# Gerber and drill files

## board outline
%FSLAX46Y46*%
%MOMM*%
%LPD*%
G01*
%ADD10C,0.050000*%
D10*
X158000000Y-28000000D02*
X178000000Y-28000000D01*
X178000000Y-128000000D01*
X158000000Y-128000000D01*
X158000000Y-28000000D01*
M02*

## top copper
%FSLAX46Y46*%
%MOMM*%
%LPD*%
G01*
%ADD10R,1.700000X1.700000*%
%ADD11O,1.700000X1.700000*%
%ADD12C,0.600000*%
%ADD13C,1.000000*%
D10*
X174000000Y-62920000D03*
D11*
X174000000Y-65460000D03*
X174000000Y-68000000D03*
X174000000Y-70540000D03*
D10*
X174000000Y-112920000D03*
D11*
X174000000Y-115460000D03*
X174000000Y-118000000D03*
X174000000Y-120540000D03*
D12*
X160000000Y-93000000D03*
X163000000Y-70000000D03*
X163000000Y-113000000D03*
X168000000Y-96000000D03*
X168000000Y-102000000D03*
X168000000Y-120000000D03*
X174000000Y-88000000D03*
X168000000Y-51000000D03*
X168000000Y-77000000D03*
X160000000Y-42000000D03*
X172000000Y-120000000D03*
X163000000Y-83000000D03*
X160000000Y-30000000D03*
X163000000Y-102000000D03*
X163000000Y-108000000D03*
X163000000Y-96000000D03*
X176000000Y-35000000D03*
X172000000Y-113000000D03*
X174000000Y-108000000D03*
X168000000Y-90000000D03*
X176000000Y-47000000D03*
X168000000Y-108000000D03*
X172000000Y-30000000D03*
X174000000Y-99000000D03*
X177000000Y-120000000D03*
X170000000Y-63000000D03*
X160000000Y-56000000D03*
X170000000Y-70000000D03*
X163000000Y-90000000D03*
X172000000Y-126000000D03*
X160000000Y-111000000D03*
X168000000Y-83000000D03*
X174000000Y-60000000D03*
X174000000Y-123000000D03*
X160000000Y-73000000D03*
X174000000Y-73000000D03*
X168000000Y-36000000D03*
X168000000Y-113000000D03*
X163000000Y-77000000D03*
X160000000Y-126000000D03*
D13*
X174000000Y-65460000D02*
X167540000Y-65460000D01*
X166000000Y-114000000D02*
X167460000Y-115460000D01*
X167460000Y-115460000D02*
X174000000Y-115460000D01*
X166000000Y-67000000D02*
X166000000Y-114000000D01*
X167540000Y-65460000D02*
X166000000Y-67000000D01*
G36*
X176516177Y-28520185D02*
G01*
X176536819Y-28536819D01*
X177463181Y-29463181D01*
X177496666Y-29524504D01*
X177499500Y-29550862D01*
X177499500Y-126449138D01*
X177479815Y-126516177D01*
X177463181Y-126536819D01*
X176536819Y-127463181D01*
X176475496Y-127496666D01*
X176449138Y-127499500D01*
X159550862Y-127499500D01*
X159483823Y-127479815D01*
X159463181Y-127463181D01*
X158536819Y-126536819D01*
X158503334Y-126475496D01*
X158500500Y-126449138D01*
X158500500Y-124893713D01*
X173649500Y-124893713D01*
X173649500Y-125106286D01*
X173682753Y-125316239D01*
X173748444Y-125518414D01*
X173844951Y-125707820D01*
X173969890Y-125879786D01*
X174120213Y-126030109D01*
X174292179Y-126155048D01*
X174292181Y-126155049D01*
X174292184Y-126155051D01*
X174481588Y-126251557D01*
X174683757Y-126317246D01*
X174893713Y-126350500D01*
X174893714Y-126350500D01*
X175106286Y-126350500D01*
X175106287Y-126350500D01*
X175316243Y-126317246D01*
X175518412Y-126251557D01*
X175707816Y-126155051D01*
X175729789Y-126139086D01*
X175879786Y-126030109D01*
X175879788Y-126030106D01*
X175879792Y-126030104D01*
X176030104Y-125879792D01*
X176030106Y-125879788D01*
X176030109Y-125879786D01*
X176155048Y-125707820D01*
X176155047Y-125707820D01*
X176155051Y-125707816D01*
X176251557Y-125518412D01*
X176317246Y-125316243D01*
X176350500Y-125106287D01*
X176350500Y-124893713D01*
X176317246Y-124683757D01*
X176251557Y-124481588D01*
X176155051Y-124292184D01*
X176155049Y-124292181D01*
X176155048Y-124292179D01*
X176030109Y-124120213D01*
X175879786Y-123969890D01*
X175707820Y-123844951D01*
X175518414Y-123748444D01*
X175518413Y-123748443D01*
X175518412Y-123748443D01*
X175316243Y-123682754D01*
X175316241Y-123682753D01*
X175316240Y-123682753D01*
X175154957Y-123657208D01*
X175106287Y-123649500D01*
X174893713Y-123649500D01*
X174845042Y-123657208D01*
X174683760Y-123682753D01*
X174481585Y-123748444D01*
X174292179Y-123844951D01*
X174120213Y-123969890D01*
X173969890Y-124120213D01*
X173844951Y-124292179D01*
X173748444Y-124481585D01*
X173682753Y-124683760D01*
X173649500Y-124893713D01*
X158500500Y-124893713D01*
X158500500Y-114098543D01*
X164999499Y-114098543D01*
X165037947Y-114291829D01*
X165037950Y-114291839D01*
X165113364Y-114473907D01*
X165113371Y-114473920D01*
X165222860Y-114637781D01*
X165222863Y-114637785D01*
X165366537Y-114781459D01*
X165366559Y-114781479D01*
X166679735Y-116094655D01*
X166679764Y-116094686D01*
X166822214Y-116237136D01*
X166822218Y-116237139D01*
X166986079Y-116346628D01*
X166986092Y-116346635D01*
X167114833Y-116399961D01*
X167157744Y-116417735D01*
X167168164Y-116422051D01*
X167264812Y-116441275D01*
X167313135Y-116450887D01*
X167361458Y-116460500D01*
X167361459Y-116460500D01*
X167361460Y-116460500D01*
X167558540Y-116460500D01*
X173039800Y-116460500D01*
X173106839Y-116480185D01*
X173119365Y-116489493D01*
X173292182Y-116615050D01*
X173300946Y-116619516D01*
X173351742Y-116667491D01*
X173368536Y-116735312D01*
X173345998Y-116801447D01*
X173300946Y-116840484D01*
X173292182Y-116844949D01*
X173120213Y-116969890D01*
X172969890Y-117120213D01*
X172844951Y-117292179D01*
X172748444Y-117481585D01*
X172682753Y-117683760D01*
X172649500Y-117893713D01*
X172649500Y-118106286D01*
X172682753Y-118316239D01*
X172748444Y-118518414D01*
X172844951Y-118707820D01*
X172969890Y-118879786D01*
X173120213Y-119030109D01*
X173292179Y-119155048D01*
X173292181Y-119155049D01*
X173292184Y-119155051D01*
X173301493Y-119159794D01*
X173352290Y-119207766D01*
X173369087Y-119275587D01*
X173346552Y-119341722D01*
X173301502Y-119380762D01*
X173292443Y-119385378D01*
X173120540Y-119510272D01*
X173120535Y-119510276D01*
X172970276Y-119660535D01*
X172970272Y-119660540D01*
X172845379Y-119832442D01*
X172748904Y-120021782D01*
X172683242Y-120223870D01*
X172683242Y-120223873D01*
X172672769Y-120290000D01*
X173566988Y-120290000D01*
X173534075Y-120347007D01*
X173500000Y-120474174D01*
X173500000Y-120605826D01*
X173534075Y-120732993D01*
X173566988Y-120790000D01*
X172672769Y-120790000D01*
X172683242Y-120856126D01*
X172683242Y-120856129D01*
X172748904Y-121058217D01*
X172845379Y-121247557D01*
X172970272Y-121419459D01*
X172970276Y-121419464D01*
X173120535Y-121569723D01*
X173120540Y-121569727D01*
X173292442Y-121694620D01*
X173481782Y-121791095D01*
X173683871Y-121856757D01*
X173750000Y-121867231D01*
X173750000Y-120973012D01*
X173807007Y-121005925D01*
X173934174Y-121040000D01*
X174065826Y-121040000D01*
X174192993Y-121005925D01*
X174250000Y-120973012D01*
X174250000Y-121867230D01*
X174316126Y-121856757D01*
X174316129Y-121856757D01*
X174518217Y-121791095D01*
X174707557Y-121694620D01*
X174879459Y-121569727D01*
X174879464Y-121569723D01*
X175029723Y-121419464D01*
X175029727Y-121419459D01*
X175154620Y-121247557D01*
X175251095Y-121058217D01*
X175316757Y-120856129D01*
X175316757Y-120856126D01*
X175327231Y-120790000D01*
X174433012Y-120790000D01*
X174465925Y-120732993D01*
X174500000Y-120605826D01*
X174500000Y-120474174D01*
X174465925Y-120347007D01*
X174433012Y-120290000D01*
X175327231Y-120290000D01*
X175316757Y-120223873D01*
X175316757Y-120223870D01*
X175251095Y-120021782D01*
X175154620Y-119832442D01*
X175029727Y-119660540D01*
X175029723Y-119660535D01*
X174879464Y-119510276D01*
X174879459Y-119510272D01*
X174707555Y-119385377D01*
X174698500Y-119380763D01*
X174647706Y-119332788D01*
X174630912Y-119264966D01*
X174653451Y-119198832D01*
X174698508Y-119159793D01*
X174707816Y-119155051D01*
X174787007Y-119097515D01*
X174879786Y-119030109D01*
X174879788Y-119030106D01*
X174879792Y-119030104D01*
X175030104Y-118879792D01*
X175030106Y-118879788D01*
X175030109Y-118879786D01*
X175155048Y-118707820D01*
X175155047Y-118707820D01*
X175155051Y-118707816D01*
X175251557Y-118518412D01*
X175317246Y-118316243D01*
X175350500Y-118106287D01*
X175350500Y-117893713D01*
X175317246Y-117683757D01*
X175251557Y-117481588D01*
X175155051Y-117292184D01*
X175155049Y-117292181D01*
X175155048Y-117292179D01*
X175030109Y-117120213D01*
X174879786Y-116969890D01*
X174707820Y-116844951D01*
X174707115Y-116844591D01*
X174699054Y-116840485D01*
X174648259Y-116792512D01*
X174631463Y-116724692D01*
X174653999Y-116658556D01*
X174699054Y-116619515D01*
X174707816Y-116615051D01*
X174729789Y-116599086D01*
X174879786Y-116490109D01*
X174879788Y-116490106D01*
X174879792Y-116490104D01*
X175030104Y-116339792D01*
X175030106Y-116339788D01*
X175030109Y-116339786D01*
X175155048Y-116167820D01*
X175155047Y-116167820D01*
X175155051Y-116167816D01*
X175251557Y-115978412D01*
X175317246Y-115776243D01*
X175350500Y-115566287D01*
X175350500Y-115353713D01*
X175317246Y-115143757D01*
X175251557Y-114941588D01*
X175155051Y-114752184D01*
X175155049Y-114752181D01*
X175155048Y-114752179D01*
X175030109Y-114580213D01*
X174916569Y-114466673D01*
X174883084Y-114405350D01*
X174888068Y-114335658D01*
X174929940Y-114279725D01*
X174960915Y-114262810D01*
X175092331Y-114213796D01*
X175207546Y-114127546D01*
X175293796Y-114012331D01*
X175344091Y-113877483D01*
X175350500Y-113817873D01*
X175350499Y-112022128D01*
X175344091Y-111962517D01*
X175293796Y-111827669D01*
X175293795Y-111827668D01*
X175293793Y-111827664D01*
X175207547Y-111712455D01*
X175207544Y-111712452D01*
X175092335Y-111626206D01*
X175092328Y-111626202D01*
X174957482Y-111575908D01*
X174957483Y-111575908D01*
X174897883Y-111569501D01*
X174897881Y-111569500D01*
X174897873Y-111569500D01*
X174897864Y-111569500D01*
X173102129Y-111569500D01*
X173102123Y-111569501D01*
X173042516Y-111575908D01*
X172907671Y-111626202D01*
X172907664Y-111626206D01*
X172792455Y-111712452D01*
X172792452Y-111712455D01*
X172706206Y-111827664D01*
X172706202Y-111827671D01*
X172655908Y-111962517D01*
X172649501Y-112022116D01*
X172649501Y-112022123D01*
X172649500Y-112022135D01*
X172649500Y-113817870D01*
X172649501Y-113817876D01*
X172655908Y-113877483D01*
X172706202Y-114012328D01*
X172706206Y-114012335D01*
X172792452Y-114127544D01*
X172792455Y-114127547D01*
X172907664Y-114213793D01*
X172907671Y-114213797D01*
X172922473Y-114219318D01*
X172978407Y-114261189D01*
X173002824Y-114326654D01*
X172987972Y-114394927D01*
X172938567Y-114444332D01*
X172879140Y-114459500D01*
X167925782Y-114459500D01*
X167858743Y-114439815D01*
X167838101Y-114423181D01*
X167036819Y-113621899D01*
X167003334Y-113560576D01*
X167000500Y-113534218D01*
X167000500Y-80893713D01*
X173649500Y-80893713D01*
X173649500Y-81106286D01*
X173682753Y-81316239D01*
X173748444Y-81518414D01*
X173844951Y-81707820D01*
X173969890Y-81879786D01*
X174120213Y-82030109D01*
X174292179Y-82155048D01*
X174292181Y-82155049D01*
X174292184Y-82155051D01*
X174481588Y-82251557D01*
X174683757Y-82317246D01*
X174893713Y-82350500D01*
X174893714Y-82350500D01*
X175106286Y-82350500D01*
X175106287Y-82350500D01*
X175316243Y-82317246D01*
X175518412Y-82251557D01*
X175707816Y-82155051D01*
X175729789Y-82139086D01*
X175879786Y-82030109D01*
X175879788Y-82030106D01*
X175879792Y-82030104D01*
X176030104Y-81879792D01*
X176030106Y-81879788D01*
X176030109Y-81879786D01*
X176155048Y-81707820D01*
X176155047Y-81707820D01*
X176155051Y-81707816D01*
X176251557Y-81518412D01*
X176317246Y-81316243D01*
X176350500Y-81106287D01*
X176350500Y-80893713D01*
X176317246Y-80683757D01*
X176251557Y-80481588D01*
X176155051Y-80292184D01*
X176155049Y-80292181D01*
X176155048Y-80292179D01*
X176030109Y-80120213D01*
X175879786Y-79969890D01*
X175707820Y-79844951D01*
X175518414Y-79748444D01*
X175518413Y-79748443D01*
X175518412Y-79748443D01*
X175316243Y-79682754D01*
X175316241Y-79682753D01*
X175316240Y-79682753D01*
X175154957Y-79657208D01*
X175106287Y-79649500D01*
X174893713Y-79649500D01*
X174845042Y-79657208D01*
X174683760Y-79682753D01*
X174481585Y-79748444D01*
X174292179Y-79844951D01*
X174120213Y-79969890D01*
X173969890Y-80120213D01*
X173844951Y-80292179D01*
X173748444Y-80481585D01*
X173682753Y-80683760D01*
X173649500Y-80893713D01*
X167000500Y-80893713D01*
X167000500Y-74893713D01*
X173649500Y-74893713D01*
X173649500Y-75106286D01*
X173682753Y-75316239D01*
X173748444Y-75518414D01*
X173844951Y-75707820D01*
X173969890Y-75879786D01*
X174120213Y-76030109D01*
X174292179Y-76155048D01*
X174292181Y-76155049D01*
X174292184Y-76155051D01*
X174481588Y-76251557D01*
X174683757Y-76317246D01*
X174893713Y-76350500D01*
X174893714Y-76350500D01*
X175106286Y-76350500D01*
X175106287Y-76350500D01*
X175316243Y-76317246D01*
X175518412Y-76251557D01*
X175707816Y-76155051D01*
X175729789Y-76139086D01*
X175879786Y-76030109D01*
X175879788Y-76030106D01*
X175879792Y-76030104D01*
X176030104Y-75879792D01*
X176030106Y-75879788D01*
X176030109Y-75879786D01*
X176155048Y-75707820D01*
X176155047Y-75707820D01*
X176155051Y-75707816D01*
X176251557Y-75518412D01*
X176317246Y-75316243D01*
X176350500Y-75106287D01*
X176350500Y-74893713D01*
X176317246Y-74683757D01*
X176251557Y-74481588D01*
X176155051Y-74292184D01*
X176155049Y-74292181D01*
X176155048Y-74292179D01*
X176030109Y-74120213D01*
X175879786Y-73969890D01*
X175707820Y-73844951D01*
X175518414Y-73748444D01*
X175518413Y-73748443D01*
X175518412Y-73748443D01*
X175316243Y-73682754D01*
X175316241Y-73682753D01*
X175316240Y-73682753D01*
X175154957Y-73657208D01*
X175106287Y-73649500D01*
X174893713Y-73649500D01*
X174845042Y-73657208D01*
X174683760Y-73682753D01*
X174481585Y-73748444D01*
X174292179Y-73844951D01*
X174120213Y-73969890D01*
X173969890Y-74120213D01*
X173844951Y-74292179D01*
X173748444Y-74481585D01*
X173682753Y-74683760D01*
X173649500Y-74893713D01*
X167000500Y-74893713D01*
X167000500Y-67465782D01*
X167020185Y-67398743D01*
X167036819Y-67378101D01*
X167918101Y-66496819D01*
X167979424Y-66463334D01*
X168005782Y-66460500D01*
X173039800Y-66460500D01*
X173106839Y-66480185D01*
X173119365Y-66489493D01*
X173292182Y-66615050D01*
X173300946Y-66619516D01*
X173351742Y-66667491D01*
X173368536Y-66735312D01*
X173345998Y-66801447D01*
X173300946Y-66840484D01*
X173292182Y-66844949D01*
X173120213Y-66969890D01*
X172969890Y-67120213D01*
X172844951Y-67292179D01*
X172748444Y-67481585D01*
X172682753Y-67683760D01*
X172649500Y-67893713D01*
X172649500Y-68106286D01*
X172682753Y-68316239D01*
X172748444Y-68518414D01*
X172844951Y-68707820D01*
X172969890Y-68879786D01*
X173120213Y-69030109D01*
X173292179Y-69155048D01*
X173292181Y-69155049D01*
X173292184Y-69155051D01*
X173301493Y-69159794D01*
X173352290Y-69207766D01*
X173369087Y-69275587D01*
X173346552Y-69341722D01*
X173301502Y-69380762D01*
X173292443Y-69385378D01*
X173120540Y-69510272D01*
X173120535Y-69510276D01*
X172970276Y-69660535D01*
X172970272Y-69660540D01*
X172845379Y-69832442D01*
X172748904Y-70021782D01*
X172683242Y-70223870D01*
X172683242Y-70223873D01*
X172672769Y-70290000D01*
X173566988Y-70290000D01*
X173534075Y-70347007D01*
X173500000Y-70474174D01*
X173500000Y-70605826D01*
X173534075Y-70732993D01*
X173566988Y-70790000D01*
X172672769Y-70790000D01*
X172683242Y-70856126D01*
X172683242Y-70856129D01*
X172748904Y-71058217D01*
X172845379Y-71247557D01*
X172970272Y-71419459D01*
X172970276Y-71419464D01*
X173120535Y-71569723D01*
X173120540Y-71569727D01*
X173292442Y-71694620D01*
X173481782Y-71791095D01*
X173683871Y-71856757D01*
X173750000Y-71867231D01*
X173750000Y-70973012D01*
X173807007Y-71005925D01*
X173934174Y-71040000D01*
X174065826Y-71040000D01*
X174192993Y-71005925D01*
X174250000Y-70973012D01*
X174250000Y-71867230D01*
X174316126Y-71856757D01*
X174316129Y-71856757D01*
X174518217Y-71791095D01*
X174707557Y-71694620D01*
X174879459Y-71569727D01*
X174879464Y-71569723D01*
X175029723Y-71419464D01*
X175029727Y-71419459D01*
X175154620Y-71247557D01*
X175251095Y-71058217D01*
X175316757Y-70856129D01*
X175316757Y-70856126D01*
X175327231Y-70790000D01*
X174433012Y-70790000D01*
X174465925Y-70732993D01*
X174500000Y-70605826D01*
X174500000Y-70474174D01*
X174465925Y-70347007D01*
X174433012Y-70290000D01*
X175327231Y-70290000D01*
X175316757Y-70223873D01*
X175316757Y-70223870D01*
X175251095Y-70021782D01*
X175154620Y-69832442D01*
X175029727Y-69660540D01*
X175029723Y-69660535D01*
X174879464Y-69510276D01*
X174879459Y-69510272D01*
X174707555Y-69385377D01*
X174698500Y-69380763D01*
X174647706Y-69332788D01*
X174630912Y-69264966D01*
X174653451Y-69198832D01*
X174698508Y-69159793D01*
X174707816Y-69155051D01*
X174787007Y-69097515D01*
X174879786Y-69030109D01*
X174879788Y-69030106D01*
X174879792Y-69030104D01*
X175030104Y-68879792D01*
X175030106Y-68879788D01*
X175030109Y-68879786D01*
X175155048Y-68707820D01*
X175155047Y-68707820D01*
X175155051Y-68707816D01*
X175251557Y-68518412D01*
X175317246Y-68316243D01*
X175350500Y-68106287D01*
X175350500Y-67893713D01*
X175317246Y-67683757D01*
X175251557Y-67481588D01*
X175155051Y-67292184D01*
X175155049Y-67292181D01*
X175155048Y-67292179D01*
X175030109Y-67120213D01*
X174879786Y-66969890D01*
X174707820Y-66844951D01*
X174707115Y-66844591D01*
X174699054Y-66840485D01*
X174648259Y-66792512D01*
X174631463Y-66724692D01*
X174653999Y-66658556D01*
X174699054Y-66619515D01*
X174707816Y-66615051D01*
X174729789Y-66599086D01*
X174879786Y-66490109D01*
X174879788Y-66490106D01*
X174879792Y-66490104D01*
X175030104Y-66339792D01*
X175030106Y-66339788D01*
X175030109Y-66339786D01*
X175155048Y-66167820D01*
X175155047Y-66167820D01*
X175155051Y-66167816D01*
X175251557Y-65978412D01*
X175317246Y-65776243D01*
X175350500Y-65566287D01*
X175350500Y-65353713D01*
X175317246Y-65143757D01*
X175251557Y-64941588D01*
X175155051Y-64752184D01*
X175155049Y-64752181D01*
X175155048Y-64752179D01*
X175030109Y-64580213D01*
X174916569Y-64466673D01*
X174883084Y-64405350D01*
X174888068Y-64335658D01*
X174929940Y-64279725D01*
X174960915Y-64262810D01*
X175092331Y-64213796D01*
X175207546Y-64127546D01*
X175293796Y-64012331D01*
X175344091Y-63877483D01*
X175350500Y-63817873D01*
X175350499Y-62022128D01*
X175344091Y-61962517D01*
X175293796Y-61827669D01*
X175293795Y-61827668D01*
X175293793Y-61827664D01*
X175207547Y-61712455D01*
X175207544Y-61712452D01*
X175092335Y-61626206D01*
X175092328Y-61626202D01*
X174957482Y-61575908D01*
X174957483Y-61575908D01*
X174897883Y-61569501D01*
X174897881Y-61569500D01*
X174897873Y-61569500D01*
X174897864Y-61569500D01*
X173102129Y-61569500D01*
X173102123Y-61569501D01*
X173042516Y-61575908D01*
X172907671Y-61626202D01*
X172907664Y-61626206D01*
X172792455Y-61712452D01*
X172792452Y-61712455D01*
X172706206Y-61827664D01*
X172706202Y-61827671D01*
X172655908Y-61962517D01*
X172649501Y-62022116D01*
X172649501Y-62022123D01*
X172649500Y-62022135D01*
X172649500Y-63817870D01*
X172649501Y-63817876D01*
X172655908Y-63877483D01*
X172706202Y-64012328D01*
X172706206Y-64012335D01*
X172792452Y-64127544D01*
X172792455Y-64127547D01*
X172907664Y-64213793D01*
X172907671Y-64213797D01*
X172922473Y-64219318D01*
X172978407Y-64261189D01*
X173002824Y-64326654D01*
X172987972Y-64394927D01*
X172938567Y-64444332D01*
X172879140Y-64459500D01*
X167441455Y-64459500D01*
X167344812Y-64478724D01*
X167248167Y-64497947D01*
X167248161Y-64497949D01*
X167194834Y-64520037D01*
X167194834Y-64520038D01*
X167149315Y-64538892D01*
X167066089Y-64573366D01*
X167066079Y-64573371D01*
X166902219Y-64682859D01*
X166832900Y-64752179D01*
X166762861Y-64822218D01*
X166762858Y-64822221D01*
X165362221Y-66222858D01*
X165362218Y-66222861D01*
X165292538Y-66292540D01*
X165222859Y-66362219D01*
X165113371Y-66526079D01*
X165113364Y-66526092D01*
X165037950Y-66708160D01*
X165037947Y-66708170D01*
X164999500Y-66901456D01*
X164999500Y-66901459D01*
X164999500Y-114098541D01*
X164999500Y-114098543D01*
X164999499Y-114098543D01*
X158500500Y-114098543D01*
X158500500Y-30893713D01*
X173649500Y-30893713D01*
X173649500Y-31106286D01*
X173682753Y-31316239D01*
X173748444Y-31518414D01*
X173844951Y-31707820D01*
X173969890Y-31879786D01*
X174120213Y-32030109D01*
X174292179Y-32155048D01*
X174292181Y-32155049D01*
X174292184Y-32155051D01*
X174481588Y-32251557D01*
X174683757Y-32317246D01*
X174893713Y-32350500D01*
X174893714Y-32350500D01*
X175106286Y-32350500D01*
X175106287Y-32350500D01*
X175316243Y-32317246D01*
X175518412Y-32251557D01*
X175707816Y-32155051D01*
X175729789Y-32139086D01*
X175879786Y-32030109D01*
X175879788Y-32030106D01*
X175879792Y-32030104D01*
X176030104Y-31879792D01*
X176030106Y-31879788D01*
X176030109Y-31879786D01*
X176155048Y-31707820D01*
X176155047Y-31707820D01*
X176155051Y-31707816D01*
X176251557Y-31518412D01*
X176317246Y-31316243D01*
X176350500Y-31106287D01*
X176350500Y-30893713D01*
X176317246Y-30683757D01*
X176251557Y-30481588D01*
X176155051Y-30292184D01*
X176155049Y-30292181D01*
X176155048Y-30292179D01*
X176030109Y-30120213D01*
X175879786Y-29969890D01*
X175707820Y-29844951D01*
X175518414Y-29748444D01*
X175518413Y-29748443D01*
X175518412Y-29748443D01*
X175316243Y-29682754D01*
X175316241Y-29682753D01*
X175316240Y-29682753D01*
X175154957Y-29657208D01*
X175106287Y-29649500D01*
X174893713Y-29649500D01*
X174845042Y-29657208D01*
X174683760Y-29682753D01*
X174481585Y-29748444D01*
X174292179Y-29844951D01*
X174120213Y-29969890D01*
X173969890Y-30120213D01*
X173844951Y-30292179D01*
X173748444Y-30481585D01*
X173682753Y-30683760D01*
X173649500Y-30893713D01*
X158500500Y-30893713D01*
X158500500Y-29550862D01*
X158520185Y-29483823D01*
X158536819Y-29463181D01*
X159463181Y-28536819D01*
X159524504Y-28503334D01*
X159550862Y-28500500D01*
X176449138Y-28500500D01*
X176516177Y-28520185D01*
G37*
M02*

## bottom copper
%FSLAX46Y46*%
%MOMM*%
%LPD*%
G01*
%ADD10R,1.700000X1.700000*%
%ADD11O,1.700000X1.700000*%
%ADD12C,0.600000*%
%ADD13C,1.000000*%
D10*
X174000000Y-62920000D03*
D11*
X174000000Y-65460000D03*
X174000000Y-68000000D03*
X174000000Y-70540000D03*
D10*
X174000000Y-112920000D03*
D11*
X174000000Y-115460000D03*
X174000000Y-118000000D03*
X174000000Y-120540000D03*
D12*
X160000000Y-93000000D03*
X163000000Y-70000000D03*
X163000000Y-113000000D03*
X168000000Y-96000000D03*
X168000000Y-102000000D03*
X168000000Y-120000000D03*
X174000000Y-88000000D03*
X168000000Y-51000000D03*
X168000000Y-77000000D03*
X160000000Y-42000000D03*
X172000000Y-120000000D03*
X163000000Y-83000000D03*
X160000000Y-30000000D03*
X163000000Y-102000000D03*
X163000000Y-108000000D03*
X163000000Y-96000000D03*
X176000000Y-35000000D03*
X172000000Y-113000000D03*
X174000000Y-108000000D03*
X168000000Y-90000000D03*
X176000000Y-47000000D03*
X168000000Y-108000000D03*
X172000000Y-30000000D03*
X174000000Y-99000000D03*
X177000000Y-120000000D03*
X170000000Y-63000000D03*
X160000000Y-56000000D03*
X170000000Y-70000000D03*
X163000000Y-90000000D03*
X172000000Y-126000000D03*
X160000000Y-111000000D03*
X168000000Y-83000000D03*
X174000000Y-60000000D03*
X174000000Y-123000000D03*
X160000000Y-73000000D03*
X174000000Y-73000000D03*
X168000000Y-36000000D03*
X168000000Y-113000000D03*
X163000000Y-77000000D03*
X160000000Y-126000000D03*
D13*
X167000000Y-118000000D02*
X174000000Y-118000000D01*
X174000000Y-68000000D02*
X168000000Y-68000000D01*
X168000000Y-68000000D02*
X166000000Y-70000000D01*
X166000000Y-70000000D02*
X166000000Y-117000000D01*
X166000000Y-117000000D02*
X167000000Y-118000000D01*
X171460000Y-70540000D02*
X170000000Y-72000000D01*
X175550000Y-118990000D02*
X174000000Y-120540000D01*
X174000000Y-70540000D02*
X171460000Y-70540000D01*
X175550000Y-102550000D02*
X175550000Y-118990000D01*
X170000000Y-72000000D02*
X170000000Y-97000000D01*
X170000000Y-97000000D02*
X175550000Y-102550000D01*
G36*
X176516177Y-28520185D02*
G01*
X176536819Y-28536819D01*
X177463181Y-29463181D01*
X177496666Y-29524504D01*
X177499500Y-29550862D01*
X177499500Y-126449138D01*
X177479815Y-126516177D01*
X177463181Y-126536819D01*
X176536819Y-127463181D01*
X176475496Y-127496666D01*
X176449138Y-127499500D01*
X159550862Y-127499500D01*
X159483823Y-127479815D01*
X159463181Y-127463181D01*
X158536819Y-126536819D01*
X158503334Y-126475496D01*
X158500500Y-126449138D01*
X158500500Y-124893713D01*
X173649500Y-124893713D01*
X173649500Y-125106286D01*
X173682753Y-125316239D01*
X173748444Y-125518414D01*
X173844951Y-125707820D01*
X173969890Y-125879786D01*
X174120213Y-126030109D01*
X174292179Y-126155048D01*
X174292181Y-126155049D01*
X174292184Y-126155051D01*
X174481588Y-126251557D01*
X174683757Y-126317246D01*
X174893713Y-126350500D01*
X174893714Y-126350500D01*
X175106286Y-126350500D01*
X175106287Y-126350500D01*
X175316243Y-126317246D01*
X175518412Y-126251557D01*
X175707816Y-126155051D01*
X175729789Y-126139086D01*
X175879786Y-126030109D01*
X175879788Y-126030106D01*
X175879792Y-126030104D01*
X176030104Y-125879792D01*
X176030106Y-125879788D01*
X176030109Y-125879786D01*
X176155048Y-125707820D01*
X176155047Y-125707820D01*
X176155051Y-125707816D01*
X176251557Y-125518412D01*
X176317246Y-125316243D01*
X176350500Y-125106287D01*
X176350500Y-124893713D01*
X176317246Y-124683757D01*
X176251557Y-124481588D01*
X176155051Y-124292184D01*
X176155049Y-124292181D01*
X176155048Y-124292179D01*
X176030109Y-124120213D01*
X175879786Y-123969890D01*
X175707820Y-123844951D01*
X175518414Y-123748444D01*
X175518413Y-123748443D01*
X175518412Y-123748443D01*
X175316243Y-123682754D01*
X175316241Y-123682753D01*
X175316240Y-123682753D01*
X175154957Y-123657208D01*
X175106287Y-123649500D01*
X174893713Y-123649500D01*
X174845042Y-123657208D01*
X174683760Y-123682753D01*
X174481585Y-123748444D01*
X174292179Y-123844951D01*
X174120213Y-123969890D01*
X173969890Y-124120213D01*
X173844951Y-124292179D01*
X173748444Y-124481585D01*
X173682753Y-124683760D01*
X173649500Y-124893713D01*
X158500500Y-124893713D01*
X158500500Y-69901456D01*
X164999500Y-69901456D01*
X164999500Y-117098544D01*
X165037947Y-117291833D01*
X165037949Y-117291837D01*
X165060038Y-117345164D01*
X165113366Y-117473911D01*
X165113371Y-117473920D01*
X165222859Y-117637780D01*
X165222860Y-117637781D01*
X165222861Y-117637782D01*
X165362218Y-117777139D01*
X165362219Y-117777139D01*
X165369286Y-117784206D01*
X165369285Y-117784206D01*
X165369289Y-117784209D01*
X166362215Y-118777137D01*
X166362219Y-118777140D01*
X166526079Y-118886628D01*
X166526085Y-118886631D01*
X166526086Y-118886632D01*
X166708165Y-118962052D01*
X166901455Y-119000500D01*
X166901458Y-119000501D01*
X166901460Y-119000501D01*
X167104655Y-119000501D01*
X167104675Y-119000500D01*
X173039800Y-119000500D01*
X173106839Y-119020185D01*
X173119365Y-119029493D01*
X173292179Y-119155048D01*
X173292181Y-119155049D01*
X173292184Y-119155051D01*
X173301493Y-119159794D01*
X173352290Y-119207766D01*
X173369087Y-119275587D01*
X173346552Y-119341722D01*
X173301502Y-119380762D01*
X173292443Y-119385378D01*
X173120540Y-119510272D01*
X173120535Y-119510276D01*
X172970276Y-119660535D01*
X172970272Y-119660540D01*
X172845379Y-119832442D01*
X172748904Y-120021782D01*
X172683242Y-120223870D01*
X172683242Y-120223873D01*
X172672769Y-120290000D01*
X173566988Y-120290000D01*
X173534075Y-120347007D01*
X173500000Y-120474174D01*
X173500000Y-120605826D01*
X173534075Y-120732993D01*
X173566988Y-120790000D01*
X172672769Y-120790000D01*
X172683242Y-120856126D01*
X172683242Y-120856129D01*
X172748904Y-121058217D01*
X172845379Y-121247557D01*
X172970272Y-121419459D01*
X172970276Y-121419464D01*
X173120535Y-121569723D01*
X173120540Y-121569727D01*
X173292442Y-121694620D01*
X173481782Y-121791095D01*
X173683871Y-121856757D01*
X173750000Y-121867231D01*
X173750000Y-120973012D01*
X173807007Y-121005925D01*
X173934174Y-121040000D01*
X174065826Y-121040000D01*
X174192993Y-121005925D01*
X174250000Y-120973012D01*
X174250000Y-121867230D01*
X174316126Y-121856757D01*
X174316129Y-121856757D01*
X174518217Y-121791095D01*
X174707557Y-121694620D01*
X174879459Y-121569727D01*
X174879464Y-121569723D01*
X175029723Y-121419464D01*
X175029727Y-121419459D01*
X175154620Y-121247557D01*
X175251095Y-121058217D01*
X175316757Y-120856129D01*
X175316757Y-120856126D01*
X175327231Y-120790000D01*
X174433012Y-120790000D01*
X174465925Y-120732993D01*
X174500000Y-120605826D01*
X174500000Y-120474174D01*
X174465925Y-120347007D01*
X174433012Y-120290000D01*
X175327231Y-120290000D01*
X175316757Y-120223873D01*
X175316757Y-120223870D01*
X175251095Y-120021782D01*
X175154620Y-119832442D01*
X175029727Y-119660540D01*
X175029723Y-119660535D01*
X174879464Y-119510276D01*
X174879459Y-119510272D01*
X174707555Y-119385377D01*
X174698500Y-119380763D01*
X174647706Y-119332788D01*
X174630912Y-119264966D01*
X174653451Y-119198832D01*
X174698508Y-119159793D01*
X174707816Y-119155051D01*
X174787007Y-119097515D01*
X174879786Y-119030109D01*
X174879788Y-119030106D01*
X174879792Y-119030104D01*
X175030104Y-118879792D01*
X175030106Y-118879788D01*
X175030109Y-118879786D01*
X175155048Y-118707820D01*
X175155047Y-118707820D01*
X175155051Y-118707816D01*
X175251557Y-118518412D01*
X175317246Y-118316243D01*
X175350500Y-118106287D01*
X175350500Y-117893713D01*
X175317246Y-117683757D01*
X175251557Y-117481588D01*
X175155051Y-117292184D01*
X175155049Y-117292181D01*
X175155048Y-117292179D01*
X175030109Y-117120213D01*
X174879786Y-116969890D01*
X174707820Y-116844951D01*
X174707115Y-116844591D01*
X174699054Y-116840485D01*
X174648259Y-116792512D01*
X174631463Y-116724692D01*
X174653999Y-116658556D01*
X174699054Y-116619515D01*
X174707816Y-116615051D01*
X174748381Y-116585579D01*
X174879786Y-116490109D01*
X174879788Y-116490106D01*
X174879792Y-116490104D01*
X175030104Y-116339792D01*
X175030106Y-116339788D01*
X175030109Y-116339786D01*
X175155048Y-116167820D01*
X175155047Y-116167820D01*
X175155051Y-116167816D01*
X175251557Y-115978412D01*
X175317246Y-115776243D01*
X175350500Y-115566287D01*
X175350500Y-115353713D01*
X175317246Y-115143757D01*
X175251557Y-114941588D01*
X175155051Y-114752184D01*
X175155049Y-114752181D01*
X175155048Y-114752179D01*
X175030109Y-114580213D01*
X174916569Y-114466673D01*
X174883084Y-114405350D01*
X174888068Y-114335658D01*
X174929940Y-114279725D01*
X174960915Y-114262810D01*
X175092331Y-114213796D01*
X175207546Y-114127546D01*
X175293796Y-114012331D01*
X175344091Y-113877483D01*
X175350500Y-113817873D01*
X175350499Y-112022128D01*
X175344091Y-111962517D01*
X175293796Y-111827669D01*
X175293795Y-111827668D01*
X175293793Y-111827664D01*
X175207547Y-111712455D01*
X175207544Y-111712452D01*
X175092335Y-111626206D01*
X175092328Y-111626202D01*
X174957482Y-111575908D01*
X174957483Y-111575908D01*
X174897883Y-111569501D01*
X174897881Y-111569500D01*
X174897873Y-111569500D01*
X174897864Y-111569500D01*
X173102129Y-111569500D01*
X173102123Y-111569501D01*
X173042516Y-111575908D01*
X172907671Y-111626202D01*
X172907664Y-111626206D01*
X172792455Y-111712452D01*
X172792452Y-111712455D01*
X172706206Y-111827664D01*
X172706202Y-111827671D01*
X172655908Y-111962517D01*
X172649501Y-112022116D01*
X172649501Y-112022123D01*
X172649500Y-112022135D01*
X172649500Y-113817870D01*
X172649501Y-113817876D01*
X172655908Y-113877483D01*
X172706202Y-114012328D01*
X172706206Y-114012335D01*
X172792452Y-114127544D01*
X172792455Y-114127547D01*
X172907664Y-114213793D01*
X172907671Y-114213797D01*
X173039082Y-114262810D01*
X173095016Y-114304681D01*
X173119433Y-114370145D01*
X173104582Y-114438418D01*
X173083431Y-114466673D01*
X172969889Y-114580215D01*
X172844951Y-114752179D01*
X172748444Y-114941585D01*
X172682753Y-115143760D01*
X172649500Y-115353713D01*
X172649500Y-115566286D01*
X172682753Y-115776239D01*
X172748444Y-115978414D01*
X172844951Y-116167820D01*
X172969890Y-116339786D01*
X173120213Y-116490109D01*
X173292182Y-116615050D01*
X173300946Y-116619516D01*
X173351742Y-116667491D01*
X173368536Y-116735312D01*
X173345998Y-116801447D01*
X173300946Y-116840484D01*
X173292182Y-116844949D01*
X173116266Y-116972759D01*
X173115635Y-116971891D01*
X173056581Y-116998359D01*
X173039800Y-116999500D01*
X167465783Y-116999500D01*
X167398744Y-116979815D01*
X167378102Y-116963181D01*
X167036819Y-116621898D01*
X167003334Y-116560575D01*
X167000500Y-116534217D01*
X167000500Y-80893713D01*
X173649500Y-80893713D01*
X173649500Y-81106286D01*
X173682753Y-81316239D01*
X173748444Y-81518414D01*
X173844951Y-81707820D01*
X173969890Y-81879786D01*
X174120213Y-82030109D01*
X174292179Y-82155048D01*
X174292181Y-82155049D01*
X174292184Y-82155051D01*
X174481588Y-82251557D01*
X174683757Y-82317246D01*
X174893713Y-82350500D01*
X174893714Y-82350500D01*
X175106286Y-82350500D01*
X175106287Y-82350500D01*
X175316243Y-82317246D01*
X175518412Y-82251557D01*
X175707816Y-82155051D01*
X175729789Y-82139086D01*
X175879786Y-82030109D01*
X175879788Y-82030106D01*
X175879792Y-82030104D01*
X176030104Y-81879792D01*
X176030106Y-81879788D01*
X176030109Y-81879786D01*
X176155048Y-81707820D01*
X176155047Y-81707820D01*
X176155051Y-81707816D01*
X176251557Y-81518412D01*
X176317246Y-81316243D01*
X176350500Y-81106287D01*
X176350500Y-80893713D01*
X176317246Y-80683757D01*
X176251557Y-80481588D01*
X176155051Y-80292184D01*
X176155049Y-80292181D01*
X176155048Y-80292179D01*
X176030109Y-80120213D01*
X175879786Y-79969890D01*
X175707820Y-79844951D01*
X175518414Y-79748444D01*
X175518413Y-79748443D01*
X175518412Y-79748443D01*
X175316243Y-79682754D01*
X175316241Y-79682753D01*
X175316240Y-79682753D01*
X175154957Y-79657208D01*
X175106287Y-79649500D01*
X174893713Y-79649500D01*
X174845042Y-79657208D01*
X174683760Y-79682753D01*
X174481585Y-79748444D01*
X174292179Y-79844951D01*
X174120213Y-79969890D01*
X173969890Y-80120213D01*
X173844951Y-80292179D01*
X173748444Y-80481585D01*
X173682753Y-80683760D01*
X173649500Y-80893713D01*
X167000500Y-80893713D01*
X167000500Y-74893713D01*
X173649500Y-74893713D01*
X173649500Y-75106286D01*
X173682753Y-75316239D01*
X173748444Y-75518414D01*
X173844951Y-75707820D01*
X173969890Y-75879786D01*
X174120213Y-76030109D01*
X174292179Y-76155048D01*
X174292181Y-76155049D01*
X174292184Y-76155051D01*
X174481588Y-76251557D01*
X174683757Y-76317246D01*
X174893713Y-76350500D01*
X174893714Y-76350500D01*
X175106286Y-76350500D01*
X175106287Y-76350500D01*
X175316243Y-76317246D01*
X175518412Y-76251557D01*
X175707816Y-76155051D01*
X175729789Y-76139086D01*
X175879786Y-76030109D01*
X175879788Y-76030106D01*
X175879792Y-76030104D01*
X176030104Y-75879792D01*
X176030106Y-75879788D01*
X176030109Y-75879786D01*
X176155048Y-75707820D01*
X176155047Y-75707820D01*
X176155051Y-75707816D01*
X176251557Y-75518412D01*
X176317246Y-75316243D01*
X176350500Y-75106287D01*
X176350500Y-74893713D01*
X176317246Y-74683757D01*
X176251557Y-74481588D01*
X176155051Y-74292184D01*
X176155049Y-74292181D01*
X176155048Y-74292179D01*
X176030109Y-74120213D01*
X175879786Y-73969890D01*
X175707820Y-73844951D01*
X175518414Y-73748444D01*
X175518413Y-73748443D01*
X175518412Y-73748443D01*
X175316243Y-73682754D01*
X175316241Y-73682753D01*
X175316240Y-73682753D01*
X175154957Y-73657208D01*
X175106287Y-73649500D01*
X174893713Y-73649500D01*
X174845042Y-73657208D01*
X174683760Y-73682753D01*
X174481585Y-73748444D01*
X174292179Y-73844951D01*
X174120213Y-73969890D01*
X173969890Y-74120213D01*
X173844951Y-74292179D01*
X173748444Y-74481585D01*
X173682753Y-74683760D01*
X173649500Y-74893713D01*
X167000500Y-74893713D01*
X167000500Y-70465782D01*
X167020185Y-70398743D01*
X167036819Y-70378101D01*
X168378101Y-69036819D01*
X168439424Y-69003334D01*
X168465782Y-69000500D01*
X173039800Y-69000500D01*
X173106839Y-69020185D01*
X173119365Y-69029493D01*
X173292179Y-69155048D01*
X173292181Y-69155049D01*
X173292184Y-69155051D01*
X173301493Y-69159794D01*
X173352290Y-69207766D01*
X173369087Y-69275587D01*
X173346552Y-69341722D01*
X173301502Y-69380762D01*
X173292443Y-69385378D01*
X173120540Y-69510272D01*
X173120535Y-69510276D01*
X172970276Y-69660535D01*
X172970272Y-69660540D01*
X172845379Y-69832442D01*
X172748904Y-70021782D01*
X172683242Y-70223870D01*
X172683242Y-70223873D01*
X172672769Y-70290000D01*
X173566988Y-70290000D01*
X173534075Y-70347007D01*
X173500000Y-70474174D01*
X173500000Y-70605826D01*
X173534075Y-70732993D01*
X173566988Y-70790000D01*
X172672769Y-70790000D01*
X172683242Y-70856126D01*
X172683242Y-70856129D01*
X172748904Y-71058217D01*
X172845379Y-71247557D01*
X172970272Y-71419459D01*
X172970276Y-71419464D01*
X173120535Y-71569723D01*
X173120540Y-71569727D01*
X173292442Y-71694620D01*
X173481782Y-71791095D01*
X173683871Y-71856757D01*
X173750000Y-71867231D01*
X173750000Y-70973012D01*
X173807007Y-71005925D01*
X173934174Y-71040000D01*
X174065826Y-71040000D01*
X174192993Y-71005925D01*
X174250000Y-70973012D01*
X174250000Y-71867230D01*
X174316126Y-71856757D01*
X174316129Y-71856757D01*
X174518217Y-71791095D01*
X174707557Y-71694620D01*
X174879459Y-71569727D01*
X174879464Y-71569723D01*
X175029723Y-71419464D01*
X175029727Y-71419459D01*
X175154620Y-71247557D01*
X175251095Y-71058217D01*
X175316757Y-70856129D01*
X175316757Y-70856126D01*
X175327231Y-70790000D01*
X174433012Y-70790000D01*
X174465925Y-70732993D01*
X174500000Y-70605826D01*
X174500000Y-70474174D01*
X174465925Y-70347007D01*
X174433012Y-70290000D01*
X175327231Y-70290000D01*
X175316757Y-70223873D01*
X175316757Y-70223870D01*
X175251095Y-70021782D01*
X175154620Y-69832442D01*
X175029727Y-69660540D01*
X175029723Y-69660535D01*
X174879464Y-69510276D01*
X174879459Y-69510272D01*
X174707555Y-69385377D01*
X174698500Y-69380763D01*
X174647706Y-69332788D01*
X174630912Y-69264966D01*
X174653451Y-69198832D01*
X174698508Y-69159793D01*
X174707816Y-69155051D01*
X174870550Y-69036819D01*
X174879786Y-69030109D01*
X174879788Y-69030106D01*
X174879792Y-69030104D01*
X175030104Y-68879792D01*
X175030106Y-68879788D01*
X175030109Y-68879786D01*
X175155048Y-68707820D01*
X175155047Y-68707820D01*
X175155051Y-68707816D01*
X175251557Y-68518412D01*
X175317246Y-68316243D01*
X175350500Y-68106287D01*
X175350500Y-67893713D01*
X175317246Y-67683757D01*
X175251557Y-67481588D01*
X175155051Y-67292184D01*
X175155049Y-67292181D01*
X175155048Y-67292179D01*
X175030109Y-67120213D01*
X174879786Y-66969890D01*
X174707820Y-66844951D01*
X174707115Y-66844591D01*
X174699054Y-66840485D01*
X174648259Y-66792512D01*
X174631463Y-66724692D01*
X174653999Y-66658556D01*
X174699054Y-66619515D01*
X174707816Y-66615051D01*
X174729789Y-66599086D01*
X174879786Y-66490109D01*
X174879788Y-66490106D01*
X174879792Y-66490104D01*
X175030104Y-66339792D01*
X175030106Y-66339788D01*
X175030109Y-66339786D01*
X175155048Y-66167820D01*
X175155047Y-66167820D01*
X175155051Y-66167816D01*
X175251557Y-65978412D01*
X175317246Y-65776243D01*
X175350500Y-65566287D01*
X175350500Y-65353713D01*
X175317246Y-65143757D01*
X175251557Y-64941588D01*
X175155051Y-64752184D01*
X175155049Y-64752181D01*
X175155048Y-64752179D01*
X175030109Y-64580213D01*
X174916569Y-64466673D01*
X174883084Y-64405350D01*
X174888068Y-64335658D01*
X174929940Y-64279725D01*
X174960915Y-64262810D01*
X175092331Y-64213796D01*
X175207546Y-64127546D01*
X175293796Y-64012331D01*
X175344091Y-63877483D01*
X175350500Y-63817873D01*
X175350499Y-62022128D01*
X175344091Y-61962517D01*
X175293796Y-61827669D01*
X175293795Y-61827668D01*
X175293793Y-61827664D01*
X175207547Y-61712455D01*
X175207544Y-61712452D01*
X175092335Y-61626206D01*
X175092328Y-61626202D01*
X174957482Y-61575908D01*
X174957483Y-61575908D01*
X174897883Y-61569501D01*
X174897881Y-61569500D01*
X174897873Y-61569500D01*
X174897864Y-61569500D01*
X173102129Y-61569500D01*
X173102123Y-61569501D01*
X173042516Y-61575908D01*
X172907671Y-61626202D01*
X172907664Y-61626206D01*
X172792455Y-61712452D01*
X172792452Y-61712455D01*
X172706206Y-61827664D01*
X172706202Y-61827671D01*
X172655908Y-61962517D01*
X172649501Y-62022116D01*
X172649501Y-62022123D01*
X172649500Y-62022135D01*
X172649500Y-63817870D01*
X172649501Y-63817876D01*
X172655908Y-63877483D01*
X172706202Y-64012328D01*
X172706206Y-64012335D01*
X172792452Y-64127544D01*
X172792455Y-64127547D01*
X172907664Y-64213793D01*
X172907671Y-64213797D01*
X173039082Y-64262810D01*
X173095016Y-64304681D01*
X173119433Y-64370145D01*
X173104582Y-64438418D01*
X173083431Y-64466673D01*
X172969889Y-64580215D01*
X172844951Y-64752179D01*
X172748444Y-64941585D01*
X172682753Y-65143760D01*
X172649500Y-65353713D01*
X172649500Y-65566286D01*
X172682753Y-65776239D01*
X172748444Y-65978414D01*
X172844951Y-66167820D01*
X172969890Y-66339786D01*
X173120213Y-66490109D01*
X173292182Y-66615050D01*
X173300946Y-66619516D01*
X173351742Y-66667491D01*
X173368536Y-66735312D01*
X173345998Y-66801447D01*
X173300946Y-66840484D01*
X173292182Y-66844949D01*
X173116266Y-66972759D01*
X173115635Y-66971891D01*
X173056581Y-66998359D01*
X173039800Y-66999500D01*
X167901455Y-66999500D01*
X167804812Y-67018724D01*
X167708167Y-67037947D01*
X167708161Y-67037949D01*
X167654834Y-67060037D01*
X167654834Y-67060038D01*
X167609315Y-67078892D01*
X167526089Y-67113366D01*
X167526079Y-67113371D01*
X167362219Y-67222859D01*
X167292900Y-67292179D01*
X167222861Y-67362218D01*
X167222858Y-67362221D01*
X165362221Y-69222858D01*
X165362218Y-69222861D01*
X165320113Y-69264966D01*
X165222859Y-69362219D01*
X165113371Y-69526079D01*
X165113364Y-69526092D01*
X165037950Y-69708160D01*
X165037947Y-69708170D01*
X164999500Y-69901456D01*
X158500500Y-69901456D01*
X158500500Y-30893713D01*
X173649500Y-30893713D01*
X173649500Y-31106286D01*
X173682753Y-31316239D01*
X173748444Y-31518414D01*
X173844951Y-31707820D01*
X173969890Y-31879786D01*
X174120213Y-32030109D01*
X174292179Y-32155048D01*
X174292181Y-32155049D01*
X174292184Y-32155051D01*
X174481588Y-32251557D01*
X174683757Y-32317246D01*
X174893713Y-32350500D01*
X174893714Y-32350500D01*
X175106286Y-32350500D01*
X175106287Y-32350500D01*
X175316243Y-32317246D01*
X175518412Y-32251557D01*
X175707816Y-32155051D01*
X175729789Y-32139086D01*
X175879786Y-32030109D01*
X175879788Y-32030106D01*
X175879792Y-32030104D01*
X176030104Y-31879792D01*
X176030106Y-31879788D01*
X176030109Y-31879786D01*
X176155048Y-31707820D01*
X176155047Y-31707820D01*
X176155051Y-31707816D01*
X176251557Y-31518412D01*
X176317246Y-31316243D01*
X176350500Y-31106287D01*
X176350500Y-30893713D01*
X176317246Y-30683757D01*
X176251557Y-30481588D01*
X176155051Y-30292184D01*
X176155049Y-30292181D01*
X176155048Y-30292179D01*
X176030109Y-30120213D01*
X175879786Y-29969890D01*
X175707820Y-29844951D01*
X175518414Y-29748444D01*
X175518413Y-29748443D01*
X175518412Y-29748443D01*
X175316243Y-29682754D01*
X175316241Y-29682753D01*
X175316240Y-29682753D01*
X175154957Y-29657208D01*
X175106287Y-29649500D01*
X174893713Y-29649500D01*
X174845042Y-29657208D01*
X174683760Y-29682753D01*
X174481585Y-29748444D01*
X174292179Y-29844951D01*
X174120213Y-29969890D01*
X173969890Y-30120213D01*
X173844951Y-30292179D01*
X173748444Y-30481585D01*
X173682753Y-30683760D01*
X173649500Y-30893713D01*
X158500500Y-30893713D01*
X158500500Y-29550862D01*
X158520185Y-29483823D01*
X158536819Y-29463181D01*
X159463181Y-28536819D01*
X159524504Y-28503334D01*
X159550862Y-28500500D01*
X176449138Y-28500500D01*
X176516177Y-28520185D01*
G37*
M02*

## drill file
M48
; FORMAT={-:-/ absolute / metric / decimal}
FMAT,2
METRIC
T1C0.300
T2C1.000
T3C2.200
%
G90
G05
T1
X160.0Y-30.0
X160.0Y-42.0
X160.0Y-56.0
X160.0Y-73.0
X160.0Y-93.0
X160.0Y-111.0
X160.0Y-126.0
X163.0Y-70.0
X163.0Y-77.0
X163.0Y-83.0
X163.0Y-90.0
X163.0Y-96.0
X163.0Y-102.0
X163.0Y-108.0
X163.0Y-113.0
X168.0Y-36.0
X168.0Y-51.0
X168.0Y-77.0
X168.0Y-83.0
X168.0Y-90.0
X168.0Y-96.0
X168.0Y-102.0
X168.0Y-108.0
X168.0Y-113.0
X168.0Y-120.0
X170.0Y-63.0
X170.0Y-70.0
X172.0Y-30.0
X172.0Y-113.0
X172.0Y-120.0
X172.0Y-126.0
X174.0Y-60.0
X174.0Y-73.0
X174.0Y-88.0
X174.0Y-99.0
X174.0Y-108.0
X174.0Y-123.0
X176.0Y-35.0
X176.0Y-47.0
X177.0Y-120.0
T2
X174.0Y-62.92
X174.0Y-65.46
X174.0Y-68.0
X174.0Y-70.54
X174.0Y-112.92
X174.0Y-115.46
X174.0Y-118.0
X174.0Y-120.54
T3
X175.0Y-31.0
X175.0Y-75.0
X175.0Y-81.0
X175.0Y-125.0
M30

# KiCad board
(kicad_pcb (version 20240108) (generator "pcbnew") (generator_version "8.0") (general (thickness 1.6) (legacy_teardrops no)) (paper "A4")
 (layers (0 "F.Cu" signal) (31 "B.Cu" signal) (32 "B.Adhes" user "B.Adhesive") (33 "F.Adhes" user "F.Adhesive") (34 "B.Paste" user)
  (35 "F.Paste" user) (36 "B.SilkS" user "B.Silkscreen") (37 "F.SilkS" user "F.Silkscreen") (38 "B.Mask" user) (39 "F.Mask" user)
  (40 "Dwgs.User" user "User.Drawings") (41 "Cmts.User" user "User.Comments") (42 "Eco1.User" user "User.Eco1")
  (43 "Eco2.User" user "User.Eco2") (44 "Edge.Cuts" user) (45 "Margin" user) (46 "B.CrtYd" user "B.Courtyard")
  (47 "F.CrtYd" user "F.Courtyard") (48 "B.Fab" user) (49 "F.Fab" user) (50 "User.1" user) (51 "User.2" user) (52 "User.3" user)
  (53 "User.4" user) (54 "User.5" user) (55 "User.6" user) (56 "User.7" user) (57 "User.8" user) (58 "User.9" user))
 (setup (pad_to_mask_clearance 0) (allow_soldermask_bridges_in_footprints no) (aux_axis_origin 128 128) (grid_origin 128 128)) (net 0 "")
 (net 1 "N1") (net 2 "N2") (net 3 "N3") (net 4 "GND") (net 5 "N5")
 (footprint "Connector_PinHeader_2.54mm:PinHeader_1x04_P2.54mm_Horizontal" (layer "F.Cu") (at 174 62.92)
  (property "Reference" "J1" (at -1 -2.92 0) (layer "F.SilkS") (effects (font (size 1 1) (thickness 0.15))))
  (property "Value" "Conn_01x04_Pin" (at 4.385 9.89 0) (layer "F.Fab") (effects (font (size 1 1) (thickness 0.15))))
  (pad "1" thru_hole rect (at 0 0) (size 1.7 1.7) (drill 1) (layers "*.Cu" "*.Mask") (remove_unused_layers no) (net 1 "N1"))
  (pad "2" thru_hole oval (at 0 2.54) (size 1.7 1.7) (drill 1) (layers "*.Cu" "*.Mask") (remove_unused_layers no) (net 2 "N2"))
  (pad "3" thru_hole oval (at 0 5.08) (size 1.7 1.7) (drill 1) (layers "*.Cu" "*.Mask") (remove_unused_layers no) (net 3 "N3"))
  (pad "4" thru_hole oval (at 0 7.62) (size 1.7 1.7) (drill 1) (layers "*.Cu" "*.Mask") (remove_unused_layers no) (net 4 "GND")))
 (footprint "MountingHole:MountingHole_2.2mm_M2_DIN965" (layer "F.Cu") (at 175 31)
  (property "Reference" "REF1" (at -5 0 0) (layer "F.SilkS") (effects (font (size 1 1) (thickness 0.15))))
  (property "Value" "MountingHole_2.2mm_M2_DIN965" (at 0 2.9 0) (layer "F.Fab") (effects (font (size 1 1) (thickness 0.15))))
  (pad "" np_thru_hole circle (at 0 0) (size 2.2 2.2) (drill 2.2) (layers "*.Cu" "*.Mask")))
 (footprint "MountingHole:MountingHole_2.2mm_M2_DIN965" (layer "F.Cu") (at 175 125)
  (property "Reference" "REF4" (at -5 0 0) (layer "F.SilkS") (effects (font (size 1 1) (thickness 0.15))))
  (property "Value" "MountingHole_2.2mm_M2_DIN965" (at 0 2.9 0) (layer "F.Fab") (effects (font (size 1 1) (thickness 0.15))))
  (pad "" np_thru_hole circle (at 0 0) (size 2.2 2.2) (drill 2.2) (layers "*.Cu" "*.Mask")))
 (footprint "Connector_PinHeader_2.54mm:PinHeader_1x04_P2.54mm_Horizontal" (layer "F.Cu") (at 174 112.92)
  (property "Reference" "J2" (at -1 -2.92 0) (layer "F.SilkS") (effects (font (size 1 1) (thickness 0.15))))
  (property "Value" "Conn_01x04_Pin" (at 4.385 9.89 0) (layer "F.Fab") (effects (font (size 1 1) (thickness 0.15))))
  (pad "1" thru_hole rect (at 0 0) (size 1.7 1.7) (drill 1) (layers "*.Cu" "*.Mask") (remove_unused_layers no) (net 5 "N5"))
  (pad "2" thru_hole oval (at 0 2.54) (size 1.7 1.7) (drill 1) (layers "*.Cu" "*.Mask") (remove_unused_layers no) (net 2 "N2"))
  (pad "3" thru_hole oval (at 0 5.08) (size 1.7 1.7) (drill 1) (layers "*.Cu" "*.Mask") (remove_unused_layers no) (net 3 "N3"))
  (pad "4" thru_hole oval (at 0 7.62) (size 1.7 1.7) (drill 1) (layers "*.Cu" "*.Mask") (remove_unused_layers no) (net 4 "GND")))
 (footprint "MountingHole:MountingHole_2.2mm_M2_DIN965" (layer "F.Cu") (at 175 75)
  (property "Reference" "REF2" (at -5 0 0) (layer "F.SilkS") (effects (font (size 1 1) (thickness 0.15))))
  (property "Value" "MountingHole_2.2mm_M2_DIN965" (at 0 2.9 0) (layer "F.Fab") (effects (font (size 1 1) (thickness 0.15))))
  (pad "" np_thru_hole circle (at 0 0) (size 2.2 2.2) (drill 2.2) (layers "*.Cu" "*.Mask")))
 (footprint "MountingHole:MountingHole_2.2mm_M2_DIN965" (layer "F.Cu") (at 175 81)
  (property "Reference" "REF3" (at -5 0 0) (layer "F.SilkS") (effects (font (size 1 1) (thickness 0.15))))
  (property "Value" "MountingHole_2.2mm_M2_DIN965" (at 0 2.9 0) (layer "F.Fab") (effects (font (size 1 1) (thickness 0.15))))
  (pad "" np_thru_hole circle (at 0 0) (size 2.2 2.2) (drill 2.2) (layers "*.Cu" "*.Mask")))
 (gr_rect (start 158 28) (end 178 128) (stroke (width 0.05) (type default)) (fill none) (layer "Edge.Cuts"))
 (segment (start 167 118) (end 174 118) (width 1) (layer "B.Cu") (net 3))
 (segment (start 174 68) (end 168 68) (width 1) (layer "B.Cu") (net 3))
 (segment (start 168 68) (end 166 70) (width 1) (layer "B.Cu") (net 3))
 (segment (start 166 70) (end 166 117) (width 1) (layer "B.Cu") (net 3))
 (segment (start 166 117) (end 167 118) (width 1) (layer "B.Cu") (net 3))
 (segment (start 174 65.46) (end 167.54 65.46) (width 1) (layer "F.Cu") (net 2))
 (segment (start 166 114) (end 167.46 115.46) (width 1) (layer "F.Cu") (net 2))
 (segment (start 167.46 115.46) (end 174 115.46) (width 1) (layer "F.Cu") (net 2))
 (segment (start 166 67) (end 166 114) (width 1) (layer "F.Cu") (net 2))
 (segment (start 167.54 65.46) (end 166 67) (width 1) (layer "F.Cu") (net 2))
 (via (at 160 93) (size 0.6) (drill 0.3) (layers "F.Cu" "B.Cu") (free yes) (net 4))
 (via (at 163 70) (size 0.6) (drill 0.3) (layers "F.Cu" "B.Cu") (free yes) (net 4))
 (via (at 163 113) (size 0.6) (drill 0.3) (layers "F.Cu" "B.Cu") (free yes) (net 4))
 (via (at 168 96) (size 0.6) (drill 0.3) (layers "F.Cu" "B.Cu") (free yes) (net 4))
 (via (at 168 102) (size 0.6) (drill 0.3) (layers "F.Cu" "B.Cu") (free yes) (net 4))
 (via (at 168 120) (size 0.6) (drill 0.3) (layers "F.Cu" "B.Cu") (free yes) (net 4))
 (via (at 174 88) (size 0.6) (drill 0.3) (layers "F.Cu" "B.Cu") (free yes) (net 4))
 (via (at 168 51) (size 0.6) (drill 0.3) (layers "F.Cu" "B.Cu") (free yes) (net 4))
 (via (at 168 77) (size 0.6) (drill 0.3) (layers "F.Cu" "B.Cu") (free yes) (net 4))
 (via (at 160 42) (size 0.6) (drill 0.3) (layers "F.Cu" "B.Cu") (free yes) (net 4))
 (via (at 172 120) (size 0.6) (drill 0.3) (layers "F.Cu" "B.Cu") (free yes) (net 4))
 (via (at 163 83) (size 0.6) (drill 0.3) (layers "F.Cu" "B.Cu") (free yes) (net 4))
 (via (at 160 30) (size 0.6) (drill 0.3) (layers "F.Cu" "B.Cu") (free yes) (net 4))
 (via (at 163 102) (size 0.6) (drill 0.3) (layers "F.Cu" "B.Cu") (free yes) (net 4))
 (via (at 163 108) (size 0.6) (drill 0.3) (layers "F.Cu" "B.Cu") (free yes) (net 4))
 (via (at 163 96) (size 0.6) (drill 0.3) (layers "F.Cu" "B.Cu") (free yes) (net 4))
 (via (at 176 35) (size 0.6) (drill 0.3) (layers "F.Cu" "B.Cu") (free yes) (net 4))
 (via (at 172 113) (size 0.6) (drill 0.3) (layers "F.Cu" "B.Cu") (free yes) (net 4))
 (via (at 174 108) (size 0.6) (drill 0.3) (layers "F.Cu" "B.Cu") (free yes) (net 4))
 (via (at 168 90) (size 0.6) (drill 0.3) (layers "F.Cu" "B.Cu") (free yes) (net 4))
 (via (at 176 47) (size 0.6) (drill 0.3) (layers "F.Cu" "B.Cu") (free yes) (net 4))
 (via (at 168 108) (size 0.6) (drill 0.3) (layers "F.Cu" "B.Cu") (free yes) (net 4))
 (via (at 172 30) (size 0.6) (drill 0.3) (layers "F.Cu" "B.Cu") (free yes) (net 4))
 (via (at 174 99) (size 0.6) (drill 0.3) (layers "F.Cu" "B.Cu") (free yes) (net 4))
 (via (at 177 120) (size 0.6) (drill 0.3) (layers "F.Cu" "B.Cu") (free yes) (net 4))
 (via (at 170 63) (size 0.6) (drill 0.3) (layers "F.Cu" "B.Cu") (free yes) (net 4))
 (via (at 160 56) (size 0.6) (drill 0.3) (layers "F.Cu" "B.Cu") (free yes) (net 4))
 (via (at 170 70) (size 0.6) (drill 0.3) (layers "F.Cu" "B.Cu") (free yes) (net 4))
 (via (at 163 90) (size 0.6) (drill 0.3) (layers "F.Cu" "B.Cu") (free yes) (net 4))
 (via (at 172 126) (size 0.6) (drill 0.3) (layers "F.Cu" "B.Cu") (free yes) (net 4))
 (via (at 160 111) (size 0.6) (drill 0.3) (layers "F.Cu" "B.Cu") (free yes) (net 4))
 (via (at 168 83) (size 0.6) (drill 0.3) (layers "F.Cu" "B.Cu") (free yes) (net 4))
 (via (at 174 60) (size 0.6) (drill 0.3) (layers "F.Cu" "B.Cu") (free yes) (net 4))
 (via (at 174 123) (size 0.6) (drill 0.3) (layers "F.Cu" "B.Cu") (free yes) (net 4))
 (via (at 160 73) (size 0.6) (drill 0.3) (layers "F.Cu" "B.Cu") (free yes) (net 4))
 (via (at 174 73) (size 0.6) (drill 0.3) (layers "F.Cu" "B.Cu") (free yes) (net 4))
 (via (at 168 36) (size 0.6) (drill 0.3) (layers "F.Cu" "B.Cu") (free yes) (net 4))
 (via (at 168 113) (size 0.6) (drill 0.3) (layers "F.Cu" "B.Cu") (free yes) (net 4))
 (via (at 163 77) (size 0.6) (drill 0.3) (layers "F.Cu" "B.Cu") (free yes) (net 4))
 (via (at 160 126) (size 0.6) (drill 0.3) (layers "F.Cu" "B.Cu") (free yes) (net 4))
 (segment (start 171.46 70.54) (end 170 72) (width 1) (layer "B.Cu") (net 4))
 (segment (start 175.55 118.99) (end 174 120.54) (width 1) (layer "B.Cu") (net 4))
 (segment (start 174 70.54) (end 171.46 70.54) (width 1) (layer "B.Cu") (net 4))
 (segment (start 175.55 102.55) (end 175.55 118.99) (width 1) (layer "B.Cu") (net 4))
 (segment (start 170 72) (end 170 97) (width 1) (layer "B.Cu") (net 4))
 (segment (start 170 97) (end 175.55 102.55) (width 1) (layer "B.Cu") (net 4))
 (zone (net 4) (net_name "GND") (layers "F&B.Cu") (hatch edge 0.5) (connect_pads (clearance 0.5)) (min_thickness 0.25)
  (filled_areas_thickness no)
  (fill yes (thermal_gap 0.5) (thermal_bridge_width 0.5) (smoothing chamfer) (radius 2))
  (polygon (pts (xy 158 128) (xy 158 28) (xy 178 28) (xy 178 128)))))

